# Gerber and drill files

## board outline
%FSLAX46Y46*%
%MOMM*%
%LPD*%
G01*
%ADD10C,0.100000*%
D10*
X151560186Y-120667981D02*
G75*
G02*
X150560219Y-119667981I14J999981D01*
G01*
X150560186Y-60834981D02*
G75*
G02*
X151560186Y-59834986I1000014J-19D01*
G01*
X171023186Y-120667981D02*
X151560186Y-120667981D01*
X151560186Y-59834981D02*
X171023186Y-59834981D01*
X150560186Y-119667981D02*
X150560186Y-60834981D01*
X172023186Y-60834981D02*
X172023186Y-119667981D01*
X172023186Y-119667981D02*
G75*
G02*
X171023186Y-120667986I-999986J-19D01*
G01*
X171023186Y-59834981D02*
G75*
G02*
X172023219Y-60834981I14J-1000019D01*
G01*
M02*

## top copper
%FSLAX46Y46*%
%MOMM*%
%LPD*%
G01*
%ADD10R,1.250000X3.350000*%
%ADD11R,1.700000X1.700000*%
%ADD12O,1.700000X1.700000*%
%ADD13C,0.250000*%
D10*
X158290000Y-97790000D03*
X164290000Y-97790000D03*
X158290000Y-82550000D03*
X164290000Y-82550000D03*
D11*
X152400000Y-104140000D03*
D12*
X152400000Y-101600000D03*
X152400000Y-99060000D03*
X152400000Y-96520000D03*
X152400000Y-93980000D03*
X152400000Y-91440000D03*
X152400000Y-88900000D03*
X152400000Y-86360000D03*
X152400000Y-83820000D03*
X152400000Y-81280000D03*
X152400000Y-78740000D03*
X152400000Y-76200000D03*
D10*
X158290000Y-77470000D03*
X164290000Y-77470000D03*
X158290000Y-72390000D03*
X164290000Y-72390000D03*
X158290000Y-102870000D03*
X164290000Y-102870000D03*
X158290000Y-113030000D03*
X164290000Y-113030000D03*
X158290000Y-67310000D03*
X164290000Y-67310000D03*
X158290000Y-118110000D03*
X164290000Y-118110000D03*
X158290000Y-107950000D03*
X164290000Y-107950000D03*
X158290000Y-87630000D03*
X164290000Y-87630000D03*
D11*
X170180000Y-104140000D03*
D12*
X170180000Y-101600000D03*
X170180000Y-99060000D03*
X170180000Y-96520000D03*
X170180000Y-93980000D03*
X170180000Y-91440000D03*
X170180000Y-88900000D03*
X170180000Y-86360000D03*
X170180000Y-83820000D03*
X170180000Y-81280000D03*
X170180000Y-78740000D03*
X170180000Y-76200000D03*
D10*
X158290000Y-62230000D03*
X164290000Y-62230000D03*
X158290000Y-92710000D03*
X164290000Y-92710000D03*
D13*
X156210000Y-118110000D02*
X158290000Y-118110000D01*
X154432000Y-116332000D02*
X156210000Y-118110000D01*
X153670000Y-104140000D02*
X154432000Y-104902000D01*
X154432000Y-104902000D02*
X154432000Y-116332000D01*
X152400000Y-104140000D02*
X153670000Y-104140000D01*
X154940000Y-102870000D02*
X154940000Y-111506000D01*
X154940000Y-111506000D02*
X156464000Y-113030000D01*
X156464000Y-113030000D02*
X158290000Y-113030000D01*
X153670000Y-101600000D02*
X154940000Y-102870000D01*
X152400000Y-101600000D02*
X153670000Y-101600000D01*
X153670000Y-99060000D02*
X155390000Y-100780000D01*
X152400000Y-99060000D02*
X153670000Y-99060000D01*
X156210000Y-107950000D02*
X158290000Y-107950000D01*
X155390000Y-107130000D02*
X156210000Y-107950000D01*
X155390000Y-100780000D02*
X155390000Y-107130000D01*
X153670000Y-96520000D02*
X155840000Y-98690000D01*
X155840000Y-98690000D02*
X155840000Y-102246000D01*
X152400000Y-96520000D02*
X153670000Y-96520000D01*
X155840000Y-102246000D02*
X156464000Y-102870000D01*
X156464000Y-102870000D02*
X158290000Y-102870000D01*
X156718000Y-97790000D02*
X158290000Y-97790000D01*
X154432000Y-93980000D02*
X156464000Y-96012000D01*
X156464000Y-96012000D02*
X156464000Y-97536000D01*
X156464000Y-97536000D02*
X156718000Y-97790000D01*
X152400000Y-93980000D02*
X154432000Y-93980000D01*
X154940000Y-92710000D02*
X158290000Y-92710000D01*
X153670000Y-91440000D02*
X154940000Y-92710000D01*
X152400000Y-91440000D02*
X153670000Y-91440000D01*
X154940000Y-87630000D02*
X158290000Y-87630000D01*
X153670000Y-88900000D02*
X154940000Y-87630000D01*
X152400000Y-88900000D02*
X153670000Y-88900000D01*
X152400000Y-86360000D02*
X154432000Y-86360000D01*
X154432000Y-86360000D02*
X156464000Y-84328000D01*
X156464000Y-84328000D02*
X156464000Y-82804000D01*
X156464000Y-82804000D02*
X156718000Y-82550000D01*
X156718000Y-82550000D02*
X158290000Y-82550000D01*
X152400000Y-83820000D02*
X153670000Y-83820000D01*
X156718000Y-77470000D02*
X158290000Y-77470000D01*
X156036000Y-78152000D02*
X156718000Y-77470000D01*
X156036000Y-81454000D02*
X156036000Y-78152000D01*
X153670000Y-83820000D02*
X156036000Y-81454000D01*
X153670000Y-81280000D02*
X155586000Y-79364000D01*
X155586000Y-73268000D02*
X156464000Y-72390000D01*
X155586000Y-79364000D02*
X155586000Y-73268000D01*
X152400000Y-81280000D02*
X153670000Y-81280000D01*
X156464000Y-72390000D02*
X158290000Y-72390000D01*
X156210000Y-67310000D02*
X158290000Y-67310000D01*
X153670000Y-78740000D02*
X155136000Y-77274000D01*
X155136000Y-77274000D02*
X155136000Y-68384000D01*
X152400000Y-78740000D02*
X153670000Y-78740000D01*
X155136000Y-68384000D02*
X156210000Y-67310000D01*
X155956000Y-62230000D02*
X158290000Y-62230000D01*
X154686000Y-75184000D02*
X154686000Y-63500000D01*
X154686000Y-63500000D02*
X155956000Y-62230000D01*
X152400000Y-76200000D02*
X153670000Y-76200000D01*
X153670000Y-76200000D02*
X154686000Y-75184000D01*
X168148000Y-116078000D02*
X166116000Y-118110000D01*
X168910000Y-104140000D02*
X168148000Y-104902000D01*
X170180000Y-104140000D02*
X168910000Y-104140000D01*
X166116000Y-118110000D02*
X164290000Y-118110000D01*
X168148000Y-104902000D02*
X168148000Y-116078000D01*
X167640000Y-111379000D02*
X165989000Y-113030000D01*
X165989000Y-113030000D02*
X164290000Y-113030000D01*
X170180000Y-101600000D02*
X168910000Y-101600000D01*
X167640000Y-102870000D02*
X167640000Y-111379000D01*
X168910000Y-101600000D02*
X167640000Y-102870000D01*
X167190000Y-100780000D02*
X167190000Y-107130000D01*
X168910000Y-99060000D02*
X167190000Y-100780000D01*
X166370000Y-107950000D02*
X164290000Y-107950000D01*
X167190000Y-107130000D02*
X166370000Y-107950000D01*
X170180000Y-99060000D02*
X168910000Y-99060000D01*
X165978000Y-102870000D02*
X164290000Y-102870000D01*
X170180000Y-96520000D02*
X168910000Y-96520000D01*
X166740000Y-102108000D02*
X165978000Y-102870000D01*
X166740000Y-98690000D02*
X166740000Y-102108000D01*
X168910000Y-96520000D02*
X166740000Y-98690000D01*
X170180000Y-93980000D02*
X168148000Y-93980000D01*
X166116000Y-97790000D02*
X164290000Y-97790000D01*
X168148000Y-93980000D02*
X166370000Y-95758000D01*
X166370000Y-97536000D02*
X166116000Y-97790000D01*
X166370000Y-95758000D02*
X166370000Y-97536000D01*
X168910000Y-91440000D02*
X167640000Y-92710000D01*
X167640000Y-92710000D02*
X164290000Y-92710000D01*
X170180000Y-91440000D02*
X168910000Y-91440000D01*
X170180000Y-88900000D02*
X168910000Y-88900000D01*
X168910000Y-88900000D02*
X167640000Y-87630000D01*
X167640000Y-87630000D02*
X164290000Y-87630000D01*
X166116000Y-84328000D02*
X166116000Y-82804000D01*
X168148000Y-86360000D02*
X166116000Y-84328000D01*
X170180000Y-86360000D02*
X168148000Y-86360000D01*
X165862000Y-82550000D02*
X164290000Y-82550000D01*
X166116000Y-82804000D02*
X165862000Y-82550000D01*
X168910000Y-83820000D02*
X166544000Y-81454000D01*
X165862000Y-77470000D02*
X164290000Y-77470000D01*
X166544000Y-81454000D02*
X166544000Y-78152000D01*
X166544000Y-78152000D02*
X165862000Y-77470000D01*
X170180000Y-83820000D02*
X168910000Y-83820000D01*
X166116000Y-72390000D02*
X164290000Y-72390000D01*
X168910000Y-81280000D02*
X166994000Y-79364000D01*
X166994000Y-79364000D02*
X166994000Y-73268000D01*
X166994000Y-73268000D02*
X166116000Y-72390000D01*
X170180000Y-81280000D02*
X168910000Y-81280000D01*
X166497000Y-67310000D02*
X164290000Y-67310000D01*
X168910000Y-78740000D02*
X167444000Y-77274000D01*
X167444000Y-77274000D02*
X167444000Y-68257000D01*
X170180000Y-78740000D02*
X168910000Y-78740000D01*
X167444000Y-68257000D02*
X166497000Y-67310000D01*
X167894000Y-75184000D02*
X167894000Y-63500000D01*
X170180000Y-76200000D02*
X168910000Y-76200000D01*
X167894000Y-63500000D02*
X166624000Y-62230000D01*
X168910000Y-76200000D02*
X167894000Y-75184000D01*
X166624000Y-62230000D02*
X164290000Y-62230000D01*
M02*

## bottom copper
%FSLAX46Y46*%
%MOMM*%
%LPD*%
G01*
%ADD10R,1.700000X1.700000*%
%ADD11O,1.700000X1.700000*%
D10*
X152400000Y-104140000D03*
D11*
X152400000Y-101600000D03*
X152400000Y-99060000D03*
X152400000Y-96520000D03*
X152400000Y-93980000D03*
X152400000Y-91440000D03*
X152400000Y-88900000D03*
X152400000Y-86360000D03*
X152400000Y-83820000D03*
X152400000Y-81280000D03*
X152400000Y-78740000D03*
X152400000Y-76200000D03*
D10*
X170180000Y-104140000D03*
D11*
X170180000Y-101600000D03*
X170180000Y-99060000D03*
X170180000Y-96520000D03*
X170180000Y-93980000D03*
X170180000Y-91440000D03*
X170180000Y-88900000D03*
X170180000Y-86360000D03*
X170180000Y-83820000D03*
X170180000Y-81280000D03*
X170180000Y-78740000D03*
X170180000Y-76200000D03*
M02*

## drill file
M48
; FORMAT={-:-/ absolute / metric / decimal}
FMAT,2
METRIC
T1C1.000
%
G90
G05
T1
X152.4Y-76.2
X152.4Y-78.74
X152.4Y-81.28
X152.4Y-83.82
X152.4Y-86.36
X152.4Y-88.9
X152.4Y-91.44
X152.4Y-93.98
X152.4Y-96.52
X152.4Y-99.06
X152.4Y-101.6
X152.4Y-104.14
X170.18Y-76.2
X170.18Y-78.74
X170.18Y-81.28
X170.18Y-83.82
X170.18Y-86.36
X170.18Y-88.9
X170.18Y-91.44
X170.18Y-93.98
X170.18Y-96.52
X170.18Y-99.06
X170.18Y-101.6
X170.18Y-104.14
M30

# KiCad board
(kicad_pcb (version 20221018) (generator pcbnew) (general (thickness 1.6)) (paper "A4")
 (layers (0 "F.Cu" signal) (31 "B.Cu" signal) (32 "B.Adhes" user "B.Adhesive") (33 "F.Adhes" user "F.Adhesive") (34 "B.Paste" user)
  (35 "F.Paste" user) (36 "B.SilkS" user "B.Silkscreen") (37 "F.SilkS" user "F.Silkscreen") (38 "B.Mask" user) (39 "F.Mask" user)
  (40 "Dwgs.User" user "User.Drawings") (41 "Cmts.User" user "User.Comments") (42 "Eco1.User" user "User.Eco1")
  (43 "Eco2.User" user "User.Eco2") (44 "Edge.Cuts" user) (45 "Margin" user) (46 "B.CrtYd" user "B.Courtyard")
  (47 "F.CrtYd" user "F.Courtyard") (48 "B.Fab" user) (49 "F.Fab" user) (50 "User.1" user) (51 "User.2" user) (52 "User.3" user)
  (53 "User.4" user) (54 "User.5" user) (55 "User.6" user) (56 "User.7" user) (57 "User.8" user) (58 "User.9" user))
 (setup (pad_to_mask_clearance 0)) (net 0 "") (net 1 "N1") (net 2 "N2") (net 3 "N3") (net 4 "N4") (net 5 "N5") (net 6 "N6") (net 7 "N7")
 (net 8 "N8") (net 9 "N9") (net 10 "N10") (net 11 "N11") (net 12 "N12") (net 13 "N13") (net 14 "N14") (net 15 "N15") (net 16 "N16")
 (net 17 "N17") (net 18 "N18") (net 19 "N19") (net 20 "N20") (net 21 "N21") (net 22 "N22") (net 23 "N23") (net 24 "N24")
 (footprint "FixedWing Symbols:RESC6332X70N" (layer "F.Cu") (at 161.29 97.79)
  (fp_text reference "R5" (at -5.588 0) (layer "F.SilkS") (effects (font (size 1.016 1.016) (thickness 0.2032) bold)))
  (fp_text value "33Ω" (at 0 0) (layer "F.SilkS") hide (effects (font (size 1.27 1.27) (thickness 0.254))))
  (pad "1" smd rect (at -3 0) (size 1.25 3.35) (layers "F.Cu" "F.Paste" "F.Mask") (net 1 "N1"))
  (pad "2" smd rect (at 3 0) (size 1.25 3.35) (layers "F.Cu" "F.Paste" "F.Mask") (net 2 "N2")))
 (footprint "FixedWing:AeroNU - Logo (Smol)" (layer "F.Cu") (at 169.026549 117.225988)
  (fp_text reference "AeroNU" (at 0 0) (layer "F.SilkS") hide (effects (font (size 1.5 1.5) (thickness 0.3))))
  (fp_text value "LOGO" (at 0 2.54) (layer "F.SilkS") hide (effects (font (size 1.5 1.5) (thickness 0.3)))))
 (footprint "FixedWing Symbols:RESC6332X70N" (layer "F.Cu") (at 161.29 82.55)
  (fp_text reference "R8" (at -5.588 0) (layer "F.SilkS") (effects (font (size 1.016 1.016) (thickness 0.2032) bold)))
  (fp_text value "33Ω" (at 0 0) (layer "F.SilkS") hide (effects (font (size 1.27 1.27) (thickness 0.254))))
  (pad "1" smd rect (at -3 0) (size 1.25 3.35) (layers "F.Cu" "F.Paste" "F.Mask") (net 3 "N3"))
  (pad "2" smd rect (at 3 0) (size 1.25 3.35) (layers "F.Cu" "F.Paste" "F.Mask") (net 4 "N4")))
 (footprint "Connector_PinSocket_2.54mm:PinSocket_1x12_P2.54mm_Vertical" (layer "F.Cu") (at 152.4 104.14 180)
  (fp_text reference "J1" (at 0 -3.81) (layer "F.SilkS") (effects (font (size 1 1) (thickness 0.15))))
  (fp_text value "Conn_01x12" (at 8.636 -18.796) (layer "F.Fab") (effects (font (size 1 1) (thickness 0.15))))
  (pad "1" thru_hole rect (at 0 0 180) (size 1.7 1.7) (drill 1) (layers "*.Cu" "*.Mask") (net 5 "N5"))
  (pad "2" thru_hole oval (at 0 2.54 180) (size 1.7 1.7) (drill 1) (layers "*.Cu" "*.Mask") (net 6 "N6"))
  (pad "3" thru_hole oval (at 0 5.08 180) (size 1.7 1.7) (drill 1) (layers "*.Cu" "*.Mask") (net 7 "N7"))
  (pad "4" thru_hole oval (at 0 7.62 180) (size 1.7 1.7) (drill 1) (layers "*.Cu" "*.Mask") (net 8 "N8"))
  (pad "5" thru_hole oval (at 0 10.16 180) (size 1.7 1.7) (drill 1) (layers "*.Cu" "*.Mask") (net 1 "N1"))
  (pad "6" thru_hole oval (at 0 12.7 180) (size 1.7 1.7) (drill 1) (layers "*.Cu" "*.Mask") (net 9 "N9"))
  (pad "7" thru_hole oval (at 0 15.24 180) (size 1.7 1.7) (drill 1) (layers "*.Cu" "*.Mask") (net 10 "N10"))
  (pad "8" thru_hole oval (at 0 17.78 180) (size 1.7 1.7) (drill 1) (layers "*.Cu" "*.Mask") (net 3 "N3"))
  (pad "9" thru_hole oval (at 0 20.32 180) (size 1.7 1.7) (drill 1) (layers "*.Cu" "*.Mask") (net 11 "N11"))
  (pad "10" thru_hole oval (at 0 22.86 180) (size 1.7 1.7) (drill 1) (layers "*.Cu" "*.Mask") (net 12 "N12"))
  (pad "11" thru_hole oval (at 0 25.4 180) (size 1.7 1.7) (drill 1) (layers "*.Cu" "*.Mask") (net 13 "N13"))
  (pad "12" thru_hole oval (at 0 27.94 180) (size 1.7 1.7) (drill 1) (layers "*.Cu" "*.Mask") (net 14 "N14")))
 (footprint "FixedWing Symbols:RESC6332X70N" (layer "F.Cu") (at 161.29 77.47)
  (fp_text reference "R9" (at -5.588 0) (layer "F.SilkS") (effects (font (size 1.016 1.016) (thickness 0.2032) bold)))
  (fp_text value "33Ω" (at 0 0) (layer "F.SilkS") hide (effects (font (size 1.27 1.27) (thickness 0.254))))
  (pad "1" smd rect (at -3 0) (size 1.25 3.35) (layers "F.Cu" "F.Paste" "F.Mask") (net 11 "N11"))
  (pad "2" smd rect (at 3 0) (size 1.25 3.35) (layers "F.Cu" "F.Paste" "F.Mask") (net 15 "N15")))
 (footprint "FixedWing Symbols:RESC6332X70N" (layer "F.Cu") (at 161.29 72.39)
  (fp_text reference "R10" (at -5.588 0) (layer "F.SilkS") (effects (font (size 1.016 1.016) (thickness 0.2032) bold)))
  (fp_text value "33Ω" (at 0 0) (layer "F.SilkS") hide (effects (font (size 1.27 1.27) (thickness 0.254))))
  (pad "1" smd rect (at -3 0) (size 1.25 3.35) (layers "F.Cu" "F.Paste" "F.Mask") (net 12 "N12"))
  (pad "2" smd rect (at 3 0) (size 1.25 3.35) (layers "F.Cu" "F.Paste" "F.Mask") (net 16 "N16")))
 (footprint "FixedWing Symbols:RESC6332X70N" (layer "F.Cu") (at 161.29 102.87)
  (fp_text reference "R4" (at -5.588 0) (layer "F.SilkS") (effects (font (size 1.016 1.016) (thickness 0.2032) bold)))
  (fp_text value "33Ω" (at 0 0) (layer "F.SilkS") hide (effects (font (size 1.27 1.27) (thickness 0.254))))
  (pad "1" smd rect (at -3 0) (size 1.25 3.35) (layers "F.Cu" "F.Paste" "F.Mask") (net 8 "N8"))
  (pad "2" smd rect (at 3 0) (size 1.25 3.35) (layers "F.Cu" "F.Paste" "F.Mask") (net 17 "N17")))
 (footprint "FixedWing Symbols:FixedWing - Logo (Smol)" (layer "F.Cu") (at 169.164 67.056 -90)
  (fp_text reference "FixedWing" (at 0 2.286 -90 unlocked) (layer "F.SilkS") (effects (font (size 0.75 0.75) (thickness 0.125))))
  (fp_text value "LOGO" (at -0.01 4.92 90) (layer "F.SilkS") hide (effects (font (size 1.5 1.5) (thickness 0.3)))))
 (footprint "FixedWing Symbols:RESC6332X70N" (layer "F.Cu") (at 161.29 113.03)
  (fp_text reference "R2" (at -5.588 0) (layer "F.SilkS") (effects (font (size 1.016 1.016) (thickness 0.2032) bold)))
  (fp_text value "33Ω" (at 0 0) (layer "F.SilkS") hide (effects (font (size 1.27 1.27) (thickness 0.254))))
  (pad "1" smd rect (at -3 0) (size 1.25 3.35) (layers "F.Cu" "F.Paste" "F.Mask") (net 6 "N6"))
  (pad "2" smd rect (at 3 0) (size 1.25 3.35) (layers "F.Cu" "F.Paste" "F.Mask") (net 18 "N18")))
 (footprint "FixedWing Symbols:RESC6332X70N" (layer "F.Cu") (at 161.29 67.31)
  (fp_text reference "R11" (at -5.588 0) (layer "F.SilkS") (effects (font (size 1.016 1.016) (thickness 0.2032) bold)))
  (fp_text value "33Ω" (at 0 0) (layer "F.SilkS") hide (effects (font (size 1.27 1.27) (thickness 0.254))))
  (pad "1" smd rect (at -3 0) (size 1.25 3.35) (layers "F.Cu" "F.Paste" "F.Mask") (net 13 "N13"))
  (pad "2" smd rect (at 3 0) (size 1.25 3.35) (layers "F.Cu" "F.Paste" "F.Mask") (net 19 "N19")))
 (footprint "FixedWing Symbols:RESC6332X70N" (layer "F.Cu") (at 161.29 118.11)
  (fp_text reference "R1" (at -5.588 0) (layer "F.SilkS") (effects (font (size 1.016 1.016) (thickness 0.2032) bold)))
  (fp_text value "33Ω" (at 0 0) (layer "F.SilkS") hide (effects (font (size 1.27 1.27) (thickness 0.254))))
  (pad "1" smd rect (at -3 0) (size 1.25 3.35) (layers "F.Cu" "F.Paste" "F.Mask") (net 5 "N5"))
  (pad "2" smd rect (at 3 0) (size 1.25 3.35) (layers "F.Cu" "F.Paste" "F.Mask") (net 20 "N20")))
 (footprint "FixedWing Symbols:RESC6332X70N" (layer "F.Cu") (at 161.29 107.95)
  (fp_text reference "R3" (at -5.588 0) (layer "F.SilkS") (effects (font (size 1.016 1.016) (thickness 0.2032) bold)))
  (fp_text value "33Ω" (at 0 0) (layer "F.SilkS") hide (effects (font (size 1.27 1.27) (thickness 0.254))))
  (pad "1" smd rect (at -3 0) (size 1.25 3.35) (layers "F.Cu" "F.Paste" "F.Mask") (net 7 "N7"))
  (pad "2" smd rect (at 3 0) (size 1.25 3.35) (layers "F.Cu" "F.Paste" "F.Mask") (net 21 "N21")))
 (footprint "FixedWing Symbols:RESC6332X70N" (layer "F.Cu") (at 161.29 87.63)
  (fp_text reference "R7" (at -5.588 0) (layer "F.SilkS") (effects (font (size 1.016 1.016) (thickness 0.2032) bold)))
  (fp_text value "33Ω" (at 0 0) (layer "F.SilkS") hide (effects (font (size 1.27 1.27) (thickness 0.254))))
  (pad "1" smd rect (at -3 0) (size 1.25 3.35) (layers "F.Cu" "F.Paste" "F.Mask") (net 10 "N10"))
  (pad "2" smd rect (at 3 0) (size 1.25 3.35) (layers "F.Cu" "F.Paste" "F.Mask") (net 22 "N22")))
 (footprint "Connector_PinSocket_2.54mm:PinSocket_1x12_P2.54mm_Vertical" (layer "F.Cu") (at 170.18 104.14 180)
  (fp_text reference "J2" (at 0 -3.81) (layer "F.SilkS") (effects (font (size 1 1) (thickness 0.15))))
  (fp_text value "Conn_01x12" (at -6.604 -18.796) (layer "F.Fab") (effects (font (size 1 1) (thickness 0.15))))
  (pad "1" thru_hole rect (at 0 0 180) (size 1.7 1.7) (drill 1) (layers "*.Cu" "*.Mask") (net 20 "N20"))
  (pad "2" thru_hole oval (at 0 2.54 180) (size 1.7 1.7) (drill 1) (layers "*.Cu" "*.Mask") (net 18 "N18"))
  (pad "3" thru_hole oval (at 0 5.08 180) (size 1.7 1.7) (drill 1) (layers "*.Cu" "*.Mask") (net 21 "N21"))
  (pad "4" thru_hole oval (at 0 7.62 180) (size 1.7 1.7) (drill 1) (layers "*.Cu" "*.Mask") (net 17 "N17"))
  (pad "5" thru_hole oval (at 0 10.16 180) (size 1.7 1.7) (drill 1) (layers "*.Cu" "*.Mask") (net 2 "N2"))
  (pad "6" thru_hole oval (at 0 12.7 180) (size 1.7 1.7) (drill 1) (layers "*.Cu" "*.Mask") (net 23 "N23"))
  (pad "7" thru_hole oval (at 0 15.24 180) (size 1.7 1.7) (drill 1) (layers "*.Cu" "*.Mask") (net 22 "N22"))
  (pad "8" thru_hole oval (at 0 17.78 180) (size 1.7 1.7) (drill 1) (layers "*.Cu" "*.Mask") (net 4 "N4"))
  (pad "9" thru_hole oval (at 0 20.32 180) (size 1.7 1.7) (drill 1) (layers "*.Cu" "*.Mask") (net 15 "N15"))
  (pad "10" thru_hole oval (at 0 22.86 180) (size 1.7 1.7) (drill 1) (layers "*.Cu" "*.Mask") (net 16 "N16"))
  (pad "11" thru_hole oval (at 0 25.4 180) (size 1.7 1.7) (drill 1) (layers "*.Cu" "*.Mask") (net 19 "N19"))
  (pad "12" thru_hole oval (at 0 27.94 180) (size 1.7 1.7) (drill 1) (layers "*.Cu" "*.Mask") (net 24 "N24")))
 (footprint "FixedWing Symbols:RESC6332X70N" (layer "F.Cu") (at 161.29 62.23)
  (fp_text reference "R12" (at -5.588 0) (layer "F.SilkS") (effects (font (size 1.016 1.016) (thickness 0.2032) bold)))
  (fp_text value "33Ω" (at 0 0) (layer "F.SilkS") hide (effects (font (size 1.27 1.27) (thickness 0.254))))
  (pad "1" smd rect (at -3 0) (size 1.25 3.35) (layers "F.Cu" "F.Paste" "F.Mask") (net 14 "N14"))
  (pad "2" smd rect (at 3 0) (size 1.25 3.35) (layers "F.Cu" "F.Paste" "F.Mask") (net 24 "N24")))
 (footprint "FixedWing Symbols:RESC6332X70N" (layer "F.Cu") (at 161.29 92.71)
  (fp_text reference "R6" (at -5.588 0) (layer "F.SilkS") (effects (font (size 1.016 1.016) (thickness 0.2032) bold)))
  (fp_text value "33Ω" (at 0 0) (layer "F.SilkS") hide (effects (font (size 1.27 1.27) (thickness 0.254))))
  (pad "1" smd rect (at -3 0) (size 1.25 3.35) (layers "F.Cu" "F.Paste" "F.Mask") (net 9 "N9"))
  (pad "2" smd rect (at 3 0) (size 1.25 3.35) (layers "F.Cu" "F.Paste" "F.Mask") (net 23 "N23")))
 (gr_arc (start 151.560186 120.667981) (mid 150.853079 120.375088) (end 150.560186 119.667981) (stroke (width 0.1) (type default))
  (layer "Edge.Cuts"))
 (gr_arc (start 150.560186 60.834981) (mid 150.853085 60.127882) (end 151.560186 59.834981) (stroke (width 0.1) (type default))
  (layer "Edge.Cuts"))
 (gr_line (start 171.023186 120.667981) (end 151.560186 120.667981) (stroke (width 0.1) (type default)) (layer "Edge.Cuts"))
 (gr_line (start 151.560186 59.834981) (end 171.023186 59.834981) (stroke (width 0.1) (type default)) (layer "Edge.Cuts"))
 (gr_line (start 150.560186 119.667981) (end 150.560186 60.834981) (stroke (width 0.1) (type default)) (layer "Edge.Cuts"))
 (gr_line (start 172.023186 60.834981) (end 172.023186 119.667981) (stroke (width 0.1) (type default)) (layer "Edge.Cuts"))
 (gr_arc (start 172.023186 119.667981) (mid 171.730299 120.375095) (end 171.023186 120.667981) (stroke (width 0.1) (type default))
  (layer "Edge.Cuts"))
 (gr_arc (start 171.023186 59.834981) (mid 171.730293 60.127874) (end 172.023186 60.834981) (stroke (width 0.1) (type default))
  (layer "Edge.Cuts"))
 (segment (start 156.21 118.11) (end 158.29 118.11) (width 0.25) (layer "F.Cu") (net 5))
 (segment (start 154.432 116.332) (end 156.21 118.11) (width 0.25) (layer "F.Cu") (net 5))
 (segment (start 153.67 104.14) (end 154.432 104.902) (width 0.25) (layer "F.Cu") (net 5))
 (segment (start 154.432 104.902) (end 154.432 116.332) (width 0.25) (layer "F.Cu") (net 5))
 (segment (start 152.4 104.14) (end 153.67 104.14) (width 0.25) (layer "F.Cu") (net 5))
 (segment (start 154.94 102.87) (end 154.94 111.506) (width 0.25) (layer "F.Cu") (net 6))
 (segment (start 154.94 111.506) (end 156.464 113.03) (width 0.25) (layer "F.Cu") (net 6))
 (segment (start 156.464 113.03) (end 158.29 113.03) (width 0.25) (layer "F.Cu") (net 6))
 (segment (start 153.67 101.6) (end 154.94 102.87) (width 0.25) (layer "F.Cu") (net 6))
 (segment (start 152.4 101.6) (end 153.67 101.6) (width 0.25) (layer "F.Cu") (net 6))
 (segment (start 153.67 99.06) (end 155.39 100.78) (width 0.25) (layer "F.Cu") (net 7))
 (segment (start 152.4 99.06) (end 153.67 99.06) (width 0.25) (layer "F.Cu") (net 7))
 (segment (start 156.21 107.95) (end 158.29 107.95) (width 0.25) (layer "F.Cu") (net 7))
 (segment (start 155.39 107.13) (end 156.21 107.95) (width 0.25) (layer "F.Cu") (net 7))
 (segment (start 155.39 100.78) (end 155.39 107.13) (width 0.25) (layer "F.Cu") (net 7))
 (segment (start 153.67 96.52) (end 155.84 98.69) (width 0.25) (layer "F.Cu") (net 8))
 (segment (start 155.84 98.69) (end 155.84 102.246) (width 0.25) (layer "F.Cu") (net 8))
 (segment (start 152.4 96.52) (end 153.67 96.52) (width 0.25) (layer "F.Cu") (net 8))
 (segment (start 155.84 102.246) (end 156.464 102.87) (width 0.25) (layer "F.Cu") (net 8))
 (segment (start 156.464 102.87) (end 158.29 102.87) (width 0.25) (layer "F.Cu") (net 8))
 (segment (start 156.718 97.79) (end 158.29 97.79) (width 0.25) (layer "F.Cu") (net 1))
 (segment (start 154.432 93.98) (end 156.464 96.012) (width 0.25) (layer "F.Cu") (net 1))
 (segment (start 156.464 96.012) (end 156.464 97.536) (width 0.25) (layer "F.Cu") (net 1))
 (segment (start 156.464 97.536) (end 156.718 97.79) (width 0.25) (layer "F.Cu") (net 1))
 (segment (start 152.4 93.98) (end 154.432 93.98) (width 0.25) (layer "F.Cu") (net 1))
 (segment (start 154.94 92.71) (end 158.29 92.71) (width 0.25) (layer "F.Cu") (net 9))
 (segment (start 153.67 91.44) (end 154.94 92.71) (width 0.25) (layer "F.Cu") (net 9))
 (segment (start 152.4 91.44) (end 153.67 91.44) (width 0.25) (layer "F.Cu") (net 9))
 (segment (start 154.94 87.63) (end 158.29 87.63) (width 0.25) (layer "F.Cu") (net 10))
 (segment (start 153.67 88.9) (end 154.94 87.63) (width 0.25) (layer "F.Cu") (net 10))
 (segment (start 152.4 88.9) (end 153.67 88.9) (width 0.25) (layer "F.Cu") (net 10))
 (segment (start 152.4 86.36) (end 154.432 86.36) (width 0.25) (layer "F.Cu") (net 3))
 (segment (start 154.432 86.36) (end 156.464 84.328) (width 0.25) (layer "F.Cu") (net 3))
 (segment (start 156.464 84.328) (end 156.464 82.804) (width 0.25) (layer "F.Cu") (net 3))
 (segment (start 156.464 82.804) (end 156.718 82.55) (width 0.25) (layer "F.Cu") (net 3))
 (segment (start 156.718 82.55) (end 158.29 82.55) (width 0.25) (layer "F.Cu") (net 3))
 (segment (start 152.4 83.82) (end 153.67 83.82) (width 0.25) (layer "F.Cu") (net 11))
 (segment (start 156.718 77.47) (end 158.29 77.47) (width 0.25) (layer "F.Cu") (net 11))
 (segment (start 156.036 78.152) (end 156.718 77.47) (width 0.25) (layer "F.Cu") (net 11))
 (segment (start 156.036 81.454) (end 156.036 78.152) (width 0.25) (layer "F.Cu") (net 11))
 (segment (start 153.67 83.82) (end 156.036 81.454) (width 0.25) (layer "F.Cu") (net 11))
 (segment (start 153.67 81.28) (end 155.586 79.364) (width 0.25) (layer "F.Cu") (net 12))
 (segment (start 155.586 73.268) (end 156.464 72.39) (width 0.25) (layer "F.Cu") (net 12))
 (segment (start 155.586 79.364) (end 155.586 73.268) (width 0.25) (layer "F.Cu") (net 12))
 (segment (start 152.4 81.28) (end 153.67 81.28) (width 0.25) (layer "F.Cu") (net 12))
 (segment (start 156.464 72.39) (end 158.29 72.39) (width 0.25) (layer "F.Cu") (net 12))
 (segment (start 156.21 67.31) (end 158.29 67.31) (width 0.25) (layer "F.Cu") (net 13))
 (segment (start 153.67 78.74) (end 155.136 77.274) (width 0.25) (layer "F.Cu") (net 13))
 (segment (start 155.136 77.274) (end 155.136 68.384) (width 0.25) (layer "F.Cu") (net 13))
 (segment (start 152.4 78.74) (end 153.67 78.74) (width 0.25) (layer "F.Cu") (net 13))
 (segment (start 155.136 68.384) (end 156.21 67.31) (width 0.25) (layer "F.Cu") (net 13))
 (segment (start 155.956 62.23) (end 158.29 62.23) (width 0.25) (layer "F.Cu") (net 14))
 (segment (start 154.686 75.184) (end 154.686 63.5) (width 0.25) (layer "F.Cu") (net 14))
 (segment (start 154.686 63.5) (end 155.956 62.23) (width 0.25) (layer "F.Cu") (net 14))
 (segment (start 152.4 76.2) (end 153.67 76.2) (width 0.25) (layer "F.Cu") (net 14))
 (segment (start 153.67 76.2) (end 154.686 75.184) (width 0.25) (layer "F.Cu") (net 14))
 (segment (start 168.148 116.078) (end 166.116 118.11) (width 0.25) (layer "F.Cu") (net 20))
 (segment (start 168.91 104.14) (end 168.148 104.902) (width 0.25) (layer "F.Cu") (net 20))
 (segment (start 170.18 104.14) (end 168.91 104.14) (width 0.25) (layer "F.Cu") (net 20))
 (segment (start 166.116 118.11) (end 164.29 118.11) (width 0.25) (layer "F.Cu") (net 20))
 (segment (start 168.148 104.902) (end 168.148 116.078) (width 0.25) (layer "F.Cu") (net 20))
 (segment (start 167.64 111.379) (end 165.989 113.03) (width 0.25) (layer "F.Cu") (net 18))
 (segment (start 165.989 113.03) (end 164.29 113.03) (width 0.25) (layer "F.Cu") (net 18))
 (segment (start 170.18 101.6) (end 168.91 101.6) (width 0.25) (layer "F.Cu") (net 18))
 (segment (start 167.64 102.87) (end 167.64 111.379) (width 0.25) (layer "F.Cu") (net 18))
 (segment (start 168.91 101.6) (end 167.64 102.87) (width 0.25) (layer "F.Cu") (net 18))
 (segment (start 167.19 100.78) (end 167.19 107.13) (width 0.25) (layer "F.Cu") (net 21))
 (segment (start 168.91 99.06) (end 167.19 100.78) (width 0.25) (layer "F.Cu") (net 21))
 (segment (start 166.37 107.95) (end 164.29 107.95) (width 0.25) (layer "F.Cu") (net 21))
 (segment (start 167.19 107.13) (end 166.37 107.95) (width 0.25) (layer "F.Cu") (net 21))
 (segment (start 170.18 99.06) (end 168.91 99.06) (width 0.25) (layer "F.Cu") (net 21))
 (segment (start 165.978 102.87) (end 164.29 102.87) (width 0.25) (layer "F.Cu") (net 17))
 (segment (start 170.18 96.52) (end 168.91 96.52) (width 0.25) (layer "F.Cu") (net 17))
 (segment (start 166.74 102.108) (end 165.978 102.87) (width 0.25) (layer "F.Cu") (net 17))
 (segment (start 166.74 98.69) (end 166.74 102.108) (width 0.25) (layer "F.Cu") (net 17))
 (segment (start 168.91 96.52) (end 166.74 98.69) (width 0.25) (layer "F.Cu") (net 17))
 (segment (start 170.18 93.98) (end 168.148 93.98) (width 0.25) (layer "F.Cu") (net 2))
 (segment (start 166.116 97.79) (end 164.29 97.79) (width 0.25) (layer "F.Cu") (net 2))
 (segment (start 168.148 93.98) (end 166.37 95.758) (width 0.25) (layer "F.Cu") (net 2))
 (segment (start 166.37 97.536) (end 166.116 97.79) (width 0.25) (layer "F.Cu") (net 2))
 (segment (start 166.37 95.758) (end 166.37 97.536) (width 0.25) (layer "F.Cu") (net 2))
 (segment (start 168.91 91.44) (end 167.64 92.71) (width 0.25) (layer "F.Cu") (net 23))
 (segment (start 167.64 92.71) (end 164.29 92.71) (width 0.25) (layer "F.Cu") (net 23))
 (segment (start 170.18 91.44) (end 168.91 91.44) (width 0.25) (layer "F.Cu") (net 23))
 (segment (start 170.18 88.9) (end 168.91 88.9) (width 0.25) (layer "F.Cu") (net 22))
 (segment (start 168.91 88.9) (end 167.64 87.63) (width 0.25) (layer "F.Cu") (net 22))
 (segment (start 167.64 87.63) (end 164.29 87.63) (width 0.25) (layer "F.Cu") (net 22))
 (segment (start 166.116 84.328) (end 166.116 82.804) (width 0.25) (layer "F.Cu") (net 4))
 (segment (start 168.148 86.36) (end 166.116 84.328) (width 0.25) (layer "F.Cu") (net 4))
 (segment (start 170.18 86.36) (end 168.148 86.36) (width 0.25) (layer "F.Cu") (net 4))
 (segment (start 165.862 82.55) (end 164.29 82.55) (width 0.25) (layer "F.Cu") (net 4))
 (segment (start 166.116 82.804) (end 165.862 82.55) (width 0.25) (layer "F.Cu") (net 4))
 (segment (start 168.91 83.82) (end 166.544 81.454) (width 0.25) (layer "F.Cu") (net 15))
 (segment (start 165.862 77.47) (end 164.29 77.47) (width 0.25) (layer "F.Cu") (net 15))
 (segment (start 166.544 81.454) (end 166.544 78.152) (width 0.25) (layer "F.Cu") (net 15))
 (segment (start 166.544 78.152) (end 165.862 77.47) (width 0.25) (layer "F.Cu") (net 15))
 (segment (start 170.18 83.82) (end 168.91 83.82) (width 0.25) (layer "F.Cu") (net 15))
 (segment (start 166.116 72.39) (end 164.29 72.39) (width 0.25) (layer "F.Cu") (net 16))
 (segment (start 168.91 81.28) (end 166.994 79.364) (width 0.25) (layer "F.Cu") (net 16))
 (segment (start 166.994 79.364) (end 166.994 73.268) (width 0.25) (layer "F.Cu") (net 16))
 (segment (start 166.994 73.268) (end 166.116 72.39) (width 0.25) (layer "F.Cu") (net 16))
 (segment (start 170.18 81.28) (end 168.91 81.28) (width 0.25) (layer "F.Cu") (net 16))
 (segment (start 166.497 67.31) (end 164.29 67.31) (width 0.25) (layer "F.Cu") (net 19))
 (segment (start 168.91 78.74) (end 167.444 77.274) (width 0.25) (layer "F.Cu") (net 19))
 (segment (start 167.444 77.274) (end 167.444 68.257) (width 0.25) (layer "F.Cu") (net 19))
 (segment (start 170.18 78.74) (end 168.91 78.74) (width 0.25) (layer "F.Cu") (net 19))
 (segment (start 167.444 68.257) (end 166.497 67.31) (width 0.25) (layer "F.Cu") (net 19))
 (segment (start 167.894 75.184) (end 167.894 63.5) (width 0.25) (layer "F.Cu") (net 24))
 (segment (start 170.18 76.2) (end 168.91 76.2) (width 0.25) (layer "F.Cu") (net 24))
 (segment (start 167.894 63.5) (end 166.624 62.23) (width 0.25) (layer "F.Cu") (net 24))
 (segment (start 168.91 76.2) (end 167.894 75.184) (width 0.25) (layer "F.Cu") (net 24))
 (segment (start 166.624 62.23) (end 164.29 62.23) (width 0.25) (layer "F.Cu") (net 24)))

